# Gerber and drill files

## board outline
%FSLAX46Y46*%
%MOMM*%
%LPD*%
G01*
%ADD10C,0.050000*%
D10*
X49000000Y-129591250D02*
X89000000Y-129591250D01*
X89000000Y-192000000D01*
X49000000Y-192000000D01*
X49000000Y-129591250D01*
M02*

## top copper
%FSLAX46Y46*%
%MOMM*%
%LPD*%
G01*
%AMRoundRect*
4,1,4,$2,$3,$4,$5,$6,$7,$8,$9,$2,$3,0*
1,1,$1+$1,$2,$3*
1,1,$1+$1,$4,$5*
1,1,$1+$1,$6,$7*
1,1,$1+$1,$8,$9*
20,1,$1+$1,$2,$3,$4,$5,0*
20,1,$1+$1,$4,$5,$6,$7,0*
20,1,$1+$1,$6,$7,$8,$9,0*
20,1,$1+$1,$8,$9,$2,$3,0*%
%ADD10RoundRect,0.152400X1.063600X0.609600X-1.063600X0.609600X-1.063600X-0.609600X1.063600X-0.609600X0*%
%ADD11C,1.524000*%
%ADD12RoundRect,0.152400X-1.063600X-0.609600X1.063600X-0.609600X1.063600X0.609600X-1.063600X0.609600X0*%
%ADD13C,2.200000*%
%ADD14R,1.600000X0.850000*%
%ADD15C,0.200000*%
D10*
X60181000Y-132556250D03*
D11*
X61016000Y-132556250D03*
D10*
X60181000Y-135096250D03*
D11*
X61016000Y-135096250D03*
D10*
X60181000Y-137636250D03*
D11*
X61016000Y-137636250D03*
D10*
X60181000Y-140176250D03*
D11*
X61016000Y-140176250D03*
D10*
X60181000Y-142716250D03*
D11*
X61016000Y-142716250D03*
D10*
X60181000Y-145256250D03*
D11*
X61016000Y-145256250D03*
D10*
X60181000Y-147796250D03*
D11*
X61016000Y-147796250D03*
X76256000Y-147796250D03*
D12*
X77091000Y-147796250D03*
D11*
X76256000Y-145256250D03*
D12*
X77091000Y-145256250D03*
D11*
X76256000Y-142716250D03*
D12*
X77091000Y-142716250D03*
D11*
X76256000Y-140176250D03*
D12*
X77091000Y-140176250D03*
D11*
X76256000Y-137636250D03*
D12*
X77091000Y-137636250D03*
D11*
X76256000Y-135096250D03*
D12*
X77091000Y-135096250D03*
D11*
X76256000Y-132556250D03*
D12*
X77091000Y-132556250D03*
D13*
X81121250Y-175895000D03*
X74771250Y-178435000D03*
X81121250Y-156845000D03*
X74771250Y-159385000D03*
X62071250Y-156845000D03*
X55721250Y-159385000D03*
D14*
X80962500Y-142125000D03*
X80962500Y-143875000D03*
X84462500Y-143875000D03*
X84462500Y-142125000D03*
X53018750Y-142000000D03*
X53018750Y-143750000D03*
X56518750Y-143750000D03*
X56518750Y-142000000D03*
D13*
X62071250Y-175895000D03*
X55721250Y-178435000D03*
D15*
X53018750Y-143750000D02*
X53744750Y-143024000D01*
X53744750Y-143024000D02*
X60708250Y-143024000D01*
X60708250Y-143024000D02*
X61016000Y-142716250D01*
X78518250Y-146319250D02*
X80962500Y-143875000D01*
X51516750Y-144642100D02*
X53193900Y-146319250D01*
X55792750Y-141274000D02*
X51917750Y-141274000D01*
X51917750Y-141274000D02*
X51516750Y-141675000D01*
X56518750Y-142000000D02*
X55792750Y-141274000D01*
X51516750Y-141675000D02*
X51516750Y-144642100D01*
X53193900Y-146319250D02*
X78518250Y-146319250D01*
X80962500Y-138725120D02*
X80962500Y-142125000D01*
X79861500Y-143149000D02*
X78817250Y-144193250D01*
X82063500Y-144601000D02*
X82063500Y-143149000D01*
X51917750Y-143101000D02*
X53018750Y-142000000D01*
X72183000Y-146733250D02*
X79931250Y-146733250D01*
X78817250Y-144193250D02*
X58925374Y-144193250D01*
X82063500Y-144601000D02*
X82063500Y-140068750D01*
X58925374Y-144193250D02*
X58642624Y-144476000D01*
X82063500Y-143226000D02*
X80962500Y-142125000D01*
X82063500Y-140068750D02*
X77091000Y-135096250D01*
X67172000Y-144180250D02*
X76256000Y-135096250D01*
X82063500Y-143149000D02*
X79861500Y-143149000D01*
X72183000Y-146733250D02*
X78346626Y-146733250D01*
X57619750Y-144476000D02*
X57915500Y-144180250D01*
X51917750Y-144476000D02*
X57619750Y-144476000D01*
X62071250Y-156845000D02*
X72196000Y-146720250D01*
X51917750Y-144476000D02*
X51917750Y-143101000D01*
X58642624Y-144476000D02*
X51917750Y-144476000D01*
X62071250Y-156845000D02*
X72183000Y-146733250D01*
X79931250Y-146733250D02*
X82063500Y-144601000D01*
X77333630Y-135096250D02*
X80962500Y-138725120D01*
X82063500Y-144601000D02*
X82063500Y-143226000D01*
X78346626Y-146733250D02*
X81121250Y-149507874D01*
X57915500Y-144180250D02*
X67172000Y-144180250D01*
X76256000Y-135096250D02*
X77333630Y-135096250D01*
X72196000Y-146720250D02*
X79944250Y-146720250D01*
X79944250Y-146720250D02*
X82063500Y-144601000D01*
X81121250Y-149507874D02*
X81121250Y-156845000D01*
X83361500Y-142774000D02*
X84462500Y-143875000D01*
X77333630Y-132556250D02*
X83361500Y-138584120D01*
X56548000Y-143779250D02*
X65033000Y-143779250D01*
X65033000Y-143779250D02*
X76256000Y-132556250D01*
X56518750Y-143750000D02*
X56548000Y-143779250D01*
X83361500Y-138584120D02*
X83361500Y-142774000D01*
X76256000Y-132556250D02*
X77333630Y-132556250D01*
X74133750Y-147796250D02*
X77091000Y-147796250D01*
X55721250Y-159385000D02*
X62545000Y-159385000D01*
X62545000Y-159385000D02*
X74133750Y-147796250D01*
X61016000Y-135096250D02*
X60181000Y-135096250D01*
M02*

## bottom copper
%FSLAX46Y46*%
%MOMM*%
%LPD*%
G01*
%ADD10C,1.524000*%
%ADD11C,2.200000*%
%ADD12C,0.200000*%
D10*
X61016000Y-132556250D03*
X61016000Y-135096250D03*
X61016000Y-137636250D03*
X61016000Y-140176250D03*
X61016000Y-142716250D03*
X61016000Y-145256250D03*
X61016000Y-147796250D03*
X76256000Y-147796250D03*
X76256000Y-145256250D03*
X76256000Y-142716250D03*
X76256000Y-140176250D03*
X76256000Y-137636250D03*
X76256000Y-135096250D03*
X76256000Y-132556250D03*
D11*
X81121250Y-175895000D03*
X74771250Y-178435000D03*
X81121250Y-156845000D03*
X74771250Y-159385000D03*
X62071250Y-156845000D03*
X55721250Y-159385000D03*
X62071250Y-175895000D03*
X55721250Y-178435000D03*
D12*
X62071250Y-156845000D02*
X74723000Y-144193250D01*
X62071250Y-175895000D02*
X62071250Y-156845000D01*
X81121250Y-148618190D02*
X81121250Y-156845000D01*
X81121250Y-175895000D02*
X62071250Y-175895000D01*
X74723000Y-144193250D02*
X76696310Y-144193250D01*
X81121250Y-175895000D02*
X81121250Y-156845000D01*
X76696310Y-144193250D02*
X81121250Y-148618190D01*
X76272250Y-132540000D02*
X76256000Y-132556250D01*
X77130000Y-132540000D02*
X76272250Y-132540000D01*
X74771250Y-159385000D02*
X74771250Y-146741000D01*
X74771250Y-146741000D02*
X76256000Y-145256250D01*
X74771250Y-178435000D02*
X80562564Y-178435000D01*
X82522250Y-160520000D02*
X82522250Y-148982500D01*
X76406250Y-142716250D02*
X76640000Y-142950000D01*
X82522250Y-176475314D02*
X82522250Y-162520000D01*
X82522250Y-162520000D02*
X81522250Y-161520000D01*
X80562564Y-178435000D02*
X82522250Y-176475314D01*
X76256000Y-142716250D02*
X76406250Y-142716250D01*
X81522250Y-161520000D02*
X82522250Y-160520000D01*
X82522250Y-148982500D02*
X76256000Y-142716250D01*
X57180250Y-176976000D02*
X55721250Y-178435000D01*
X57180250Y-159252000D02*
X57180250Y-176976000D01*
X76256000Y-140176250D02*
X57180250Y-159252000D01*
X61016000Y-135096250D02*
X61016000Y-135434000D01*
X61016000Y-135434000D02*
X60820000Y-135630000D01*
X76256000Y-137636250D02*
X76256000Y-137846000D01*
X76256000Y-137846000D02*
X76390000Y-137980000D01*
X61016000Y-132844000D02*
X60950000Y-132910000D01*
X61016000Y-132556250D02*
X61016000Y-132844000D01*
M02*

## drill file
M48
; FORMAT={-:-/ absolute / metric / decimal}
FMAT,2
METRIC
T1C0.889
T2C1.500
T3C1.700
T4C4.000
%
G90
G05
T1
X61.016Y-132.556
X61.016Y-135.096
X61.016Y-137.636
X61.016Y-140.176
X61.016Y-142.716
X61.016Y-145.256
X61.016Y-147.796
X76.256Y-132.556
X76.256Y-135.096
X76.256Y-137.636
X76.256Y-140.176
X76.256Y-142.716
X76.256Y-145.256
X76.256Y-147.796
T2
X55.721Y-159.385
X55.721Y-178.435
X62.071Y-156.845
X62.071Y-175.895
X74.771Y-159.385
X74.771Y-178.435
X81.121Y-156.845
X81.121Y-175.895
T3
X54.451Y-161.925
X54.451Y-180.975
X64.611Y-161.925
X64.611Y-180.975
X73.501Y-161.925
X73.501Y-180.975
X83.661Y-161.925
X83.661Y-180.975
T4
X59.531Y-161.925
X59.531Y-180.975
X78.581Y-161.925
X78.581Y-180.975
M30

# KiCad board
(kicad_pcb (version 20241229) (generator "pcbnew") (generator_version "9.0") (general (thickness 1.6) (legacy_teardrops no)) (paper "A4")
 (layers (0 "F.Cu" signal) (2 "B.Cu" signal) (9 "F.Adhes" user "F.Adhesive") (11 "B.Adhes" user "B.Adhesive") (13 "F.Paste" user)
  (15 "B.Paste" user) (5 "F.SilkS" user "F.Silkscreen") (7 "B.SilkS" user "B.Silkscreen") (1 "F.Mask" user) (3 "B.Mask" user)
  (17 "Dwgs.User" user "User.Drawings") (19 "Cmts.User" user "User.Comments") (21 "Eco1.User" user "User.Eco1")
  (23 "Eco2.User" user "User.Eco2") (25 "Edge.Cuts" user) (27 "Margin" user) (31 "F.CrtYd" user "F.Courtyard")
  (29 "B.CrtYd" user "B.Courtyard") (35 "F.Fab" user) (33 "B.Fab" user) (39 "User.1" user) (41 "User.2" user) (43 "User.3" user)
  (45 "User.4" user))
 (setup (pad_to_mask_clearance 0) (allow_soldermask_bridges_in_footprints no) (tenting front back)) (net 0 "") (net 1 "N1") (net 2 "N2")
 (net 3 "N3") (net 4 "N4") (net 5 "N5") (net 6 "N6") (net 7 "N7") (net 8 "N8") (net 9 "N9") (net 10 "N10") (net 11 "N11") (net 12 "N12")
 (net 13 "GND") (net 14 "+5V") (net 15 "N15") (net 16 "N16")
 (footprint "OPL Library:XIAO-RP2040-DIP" (layer "F.Cu") (at 68.636 140.17625)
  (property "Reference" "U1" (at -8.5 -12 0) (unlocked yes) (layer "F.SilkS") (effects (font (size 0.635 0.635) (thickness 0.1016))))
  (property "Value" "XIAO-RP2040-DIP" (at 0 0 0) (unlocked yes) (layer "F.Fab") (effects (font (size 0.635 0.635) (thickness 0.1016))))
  (pad "1" smd roundrect (at -8.455 -7.62 180) (size 2.432 1.524) (layers "F.Cu" "F.Mask") (roundrect_rratio 0.1) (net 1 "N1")
   (thermal_bridge_angle 45))
  (pad "1" thru_hole circle (at -7.62 -7.62 180) (size 1.524 1.524) (drill 0.889) (layers "*.Cu" "*.Mask") (remove_unused_layers no)
   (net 1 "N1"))
  (pad "2" smd roundrect (at -8.455 -5.08 180) (size 2.432 1.524) (layers "F.Cu" "F.Mask") (roundrect_rratio 0.1) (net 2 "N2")
   (thermal_bridge_angle 45))
  (pad "2" thru_hole circle (at -7.62 -5.08 180) (size 1.524 1.524) (drill 0.889) (layers "*.Cu" "*.Mask") (remove_unused_layers no)
   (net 2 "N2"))
  (pad "3" smd roundrect (at -8.455 -2.54 180) (size 2.432 1.524) (layers "F.Cu" "F.Mask") (roundrect_rratio 0.1) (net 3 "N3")
   (thermal_bridge_angle 45))
  (pad "3" thru_hole circle (at -7.62 -2.54 180) (size 1.524 1.524) (drill 0.889) (layers "*.Cu" "*.Mask") (remove_unused_layers no)
   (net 3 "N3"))
  (pad "4" smd roundrect (at -8.455 0 180) (size 2.432 1.524) (layers "F.Cu" "F.Mask") (roundrect_rratio 0.1) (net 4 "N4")
   (thermal_bridge_angle 45))
  (pad "4" thru_hole circle (at -7.62 0 180) (size 1.524 1.524) (drill 0.889) (layers "*.Cu" "*.Mask") (remove_unused_layers no)
   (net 4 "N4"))
  (pad "5" smd roundrect (at -8.455 2.54 180) (size 2.432 1.524) (layers "F.Cu" "F.Mask") (roundrect_rratio 0.1) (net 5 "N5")
   (thermal_bridge_angle 45))
  (pad "5" thru_hole circle (at -7.62 2.54 180) (size 1.524 1.524) (drill 0.889) (layers "*.Cu" "*.Mask") (remove_unused_layers no)
   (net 5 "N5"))
  (pad "6" smd roundrect (at -8.455 5.08 180) (size 2.432 1.524) (layers "F.Cu" "F.Mask") (roundrect_rratio 0.1) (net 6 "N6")
   (thermal_bridge_angle 45))
  (pad "6" thru_hole circle (at -7.62 5.08 180) (size 1.524 1.524) (drill 0.889) (layers "*.Cu" "*.Mask") (remove_unused_layers no)
   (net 6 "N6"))
  (pad "7" smd roundrect (at -8.455 7.62 180) (size 2.432 1.524) (layers "F.Cu" "F.Mask") (roundrect_rratio 0.1) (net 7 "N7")
   (thermal_bridge_angle 45))
  (pad "7" thru_hole circle (at -7.62 7.62 180) (size 1.524 1.524) (drill 0.889) (layers "*.Cu" "*.Mask") (remove_unused_layers no)
   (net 7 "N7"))
  (pad "8" thru_hole circle (at 7.62 7.62) (size 1.524 1.524) (drill 0.889) (layers "*.Cu" "*.Mask") (remove_unused_layers no) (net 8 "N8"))
  (pad "8" smd roundrect (at 8.455 7.62) (size 2.432 1.524) (layers "F.Cu" "F.Mask") (roundrect_rratio 0.1) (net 8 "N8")
   (thermal_bridge_angle 45))
  (pad "9" thru_hole circle (at 7.62 5.08) (size 1.524 1.524) (drill 0.889) (layers "*.Cu" "*.Mask") (remove_unused_layers no) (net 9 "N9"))
  (pad "9" smd roundrect (at 8.455 5.08) (size 2.432 1.524) (layers "F.Cu" "F.Mask") (roundrect_rratio 0.1) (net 9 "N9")
   (thermal_bridge_angle 45))
  (pad "10" thru_hole circle (at 7.62 2.54) (size 1.524 1.524) (drill 0.889) (layers "*.Cu" "*.Mask") (remove_unused_layers no)
   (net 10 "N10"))
  (pad "10" smd roundrect (at 8.455 2.54) (size 2.432 1.524) (layers "F.Cu" "F.Mask") (roundrect_rratio 0.1) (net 10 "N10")
   (thermal_bridge_angle 45))
  (pad "11" thru_hole circle (at 7.62 0) (size 1.524 1.524) (drill 0.889) (layers "*.Cu" "*.Mask") (remove_unused_layers no) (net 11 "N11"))
  (pad "11" smd roundrect (at 8.455 0) (size 2.432 1.524) (layers "F.Cu" "F.Mask") (roundrect_rratio 0.1) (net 11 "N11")
   (thermal_bridge_angle 45))
  (pad "12" thru_hole circle (at 7.62 -2.54) (size 1.524 1.524) (drill 0.889) (layers "*.Cu" "*.Mask") (remove_unused_layers no)
   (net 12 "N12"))
  (pad "12" smd roundrect (at 8.455 -2.54) (size 2.432 1.524) (layers "F.Cu" "F.Mask") (roundrect_rratio 0.1) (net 12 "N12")
   (thermal_bridge_angle 45))
  (pad "13" thru_hole circle (at 7.62 -5.08) (size 1.524 1.524) (drill 0.889) (layers "*.Cu" "*.Mask") (remove_unused_layers no)
   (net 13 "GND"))
  (pad "13" smd roundrect (at 8.455 -5.08) (size 2.432 1.524) (layers "F.Cu" "F.Mask") (roundrect_rratio 0.1) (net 13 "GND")
   (thermal_bridge_angle 45))
  (pad "14" thru_hole circle (at 7.62 -7.62) (size 1.524 1.524) (drill 0.889) (layers "*.Cu" "*.Mask") (remove_unused_layers no)
   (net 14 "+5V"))
  (pad "14" smd roundrect (at 8.455 -7.62) (size 2.432 1.524) (layers "F.Cu" "F.Mask") (roundrect_rratio 0.1) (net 14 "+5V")
   (thermal_bridge_angle 45)))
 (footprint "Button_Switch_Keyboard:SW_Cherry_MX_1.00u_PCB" (layer "F.Cu") (at 81.12125 175.895)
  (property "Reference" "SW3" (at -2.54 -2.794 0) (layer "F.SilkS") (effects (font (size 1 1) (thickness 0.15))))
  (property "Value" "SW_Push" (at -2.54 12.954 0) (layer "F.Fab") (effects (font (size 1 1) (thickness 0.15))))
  (pad "" np_thru_hole circle (at -7.62 5.08) (size 1.7 1.7) (drill 1.7) (layers "*.Cu" "*.Mask"))
  (pad "" np_thru_hole circle (at -2.54 5.08) (size 4 4) (drill 4) (layers "*.Cu" "*.Mask"))
  (pad "" np_thru_hole circle (at 2.54 5.08) (size 1.7 1.7) (drill 1.7) (layers "*.Cu" "*.Mask"))
  (pad "1" thru_hole circle (at 0 0) (size 2.2 2.2) (drill 1.5) (layers "*.Cu" "*.Mask") (remove_unused_layers no) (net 13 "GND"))
  (pad "2" thru_hole circle (at -6.35 2.54) (size 2.2 2.2) (drill 1.5) (layers "*.Cu" "*.Mask") (remove_unused_layers no) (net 10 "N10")))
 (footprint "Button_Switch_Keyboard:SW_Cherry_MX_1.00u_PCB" (layer "F.Cu") (at 81.12125 156.845)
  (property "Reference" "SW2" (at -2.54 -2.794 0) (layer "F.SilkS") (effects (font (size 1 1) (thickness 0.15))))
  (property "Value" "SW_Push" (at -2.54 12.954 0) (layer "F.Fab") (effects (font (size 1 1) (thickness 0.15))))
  (pad "" np_thru_hole circle (at -7.62 5.08) (size 1.7 1.7) (drill 1.7) (layers "*.Cu" "*.Mask"))
  (pad "" np_thru_hole circle (at -2.54 5.08) (size 4 4) (drill 4) (layers "*.Cu" "*.Mask"))
  (pad "" np_thru_hole circle (at 2.54 5.08) (size 1.7 1.7) (drill 1.7) (layers "*.Cu" "*.Mask"))
  (pad "1" thru_hole circle (at 0 0) (size 2.2 2.2) (drill 1.5) (layers "*.Cu" "*.Mask") (remove_unused_layers no) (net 13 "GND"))
  (pad "2" thru_hole circle (at -6.35 2.54) (size 2.2 2.2) (drill 1.5) (layers "*.Cu" "*.Mask") (remove_unused_layers no) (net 9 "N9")))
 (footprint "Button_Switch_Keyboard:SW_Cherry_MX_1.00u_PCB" (layer "F.Cu") (at 62.07125 156.845)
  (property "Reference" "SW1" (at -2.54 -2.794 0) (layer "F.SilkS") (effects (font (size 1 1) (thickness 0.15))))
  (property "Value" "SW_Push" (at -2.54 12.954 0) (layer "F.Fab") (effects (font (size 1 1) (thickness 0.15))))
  (pad "" np_thru_hole circle (at -7.62 5.08) (size 1.7 1.7) (drill 1.7) (layers "*.Cu" "*.Mask"))
  (pad "" np_thru_hole circle (at -2.54 5.08) (size 4 4) (drill 4) (layers "*.Cu" "*.Mask"))
  (pad "" np_thru_hole circle (at 2.54 5.08) (size 1.7 1.7) (drill 1.7) (layers "*.Cu" "*.Mask"))
  (pad "1" thru_hole circle (at 0 0) (size 2.2 2.2) (drill 1.5) (layers "*.Cu" "*.Mask") (remove_unused_layers no) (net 13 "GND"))
  (pad "2" thru_hole circle (at -6.35 2.54) (size 2.2 2.2) (drill 1.5) (layers "*.Cu" "*.Mask") (remove_unused_layers no) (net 8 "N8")))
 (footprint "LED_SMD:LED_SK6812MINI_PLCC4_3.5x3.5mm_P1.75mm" (layer "F.Cu") (at 82.7125 143)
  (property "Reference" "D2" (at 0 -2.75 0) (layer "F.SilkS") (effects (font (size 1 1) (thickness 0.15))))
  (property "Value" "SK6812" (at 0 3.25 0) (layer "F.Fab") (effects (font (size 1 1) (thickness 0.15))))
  (pad "1" smd rect (at -1.75 -0.875) (size 1.6 0.85) (layers "F.Cu" "F.Mask" "F.Paste") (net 13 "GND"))
  (pad "2" smd rect (at -1.75 0.875) (size 1.6 0.85) (layers "F.Cu" "F.Mask" "F.Paste") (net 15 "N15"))
  (pad "3" smd rect (at 1.75 0.875) (size 1.6 0.85) (layers "F.Cu" "F.Mask" "F.Paste") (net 14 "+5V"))
  (pad "4" smd rect (at 1.75 -0.875) (size 1.6 0.85) (layers "F.Cu" "F.Mask" "F.Paste") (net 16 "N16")))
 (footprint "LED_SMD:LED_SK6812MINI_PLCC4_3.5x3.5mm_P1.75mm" (layer "F.Cu") (at 54.76875 142.875)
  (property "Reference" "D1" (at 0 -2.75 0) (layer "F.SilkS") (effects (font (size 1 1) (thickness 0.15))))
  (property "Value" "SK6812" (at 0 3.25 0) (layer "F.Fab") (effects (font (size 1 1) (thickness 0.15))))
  (pad "1" smd rect (at -1.75 -0.875) (size 1.6 0.85) (layers "F.Cu" "F.Mask" "F.Paste") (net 13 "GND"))
  (pad "2" smd rect (at -1.75 0.875) (size 1.6 0.85) (layers "F.Cu" "F.Mask" "F.Paste") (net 5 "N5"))
  (pad "3" smd rect (at 1.75 0.875) (size 1.6 0.85) (layers "F.Cu" "F.Mask" "F.Paste") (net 14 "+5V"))
  (pad "4" smd rect (at 1.75 -0.875) (size 1.6 0.85) (layers "F.Cu" "F.Mask" "F.Paste") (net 15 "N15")))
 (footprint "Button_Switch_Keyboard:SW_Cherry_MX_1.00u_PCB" (layer "F.Cu") (at 62.07125 175.895)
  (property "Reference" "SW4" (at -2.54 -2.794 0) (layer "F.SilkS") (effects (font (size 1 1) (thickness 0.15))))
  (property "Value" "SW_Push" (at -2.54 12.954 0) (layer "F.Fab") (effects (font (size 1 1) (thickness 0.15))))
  (pad "" np_thru_hole circle (at -7.62 5.08) (size 1.7 1.7) (drill 1.7) (layers "*.Cu" "*.Mask"))
  (pad "" np_thru_hole circle (at -2.54 5.08) (size 4 4) (drill 4) (layers "*.Cu" "*.Mask"))
  (pad "" np_thru_hole circle (at 2.54 5.08) (size 1.7 1.7) (drill 1.7) (layers "*.Cu" "*.Mask"))
  (pad "1" thru_hole circle (at 0 0) (size 2.2 2.2) (drill 1.5) (layers "*.Cu" "*.Mask") (remove_unused_layers no) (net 13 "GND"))
  (pad "2" thru_hole circle (at -6.35 2.54) (size 2.2 2.2) (drill 1.5) (layers "*.Cu" "*.Mask") (remove_unused_layers no) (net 11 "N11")))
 (gr_rect (start 49 129.59125) (end 89 192) (stroke (width 0.05) (type default)) (fill no) (layer "Edge.Cuts"))
 (segment (start 53.01875 143.75) (end 53.74475 143.024) (width 0.2) (layer "F.Cu") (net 5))
 (segment (start 53.74475 143.024) (end 60.70825 143.024) (width 0.2) (layer "F.Cu") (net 5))
 (segment (start 60.70825 143.024) (end 61.016 142.71625) (width 0.2) (layer "F.Cu") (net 5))
 (segment (start 78.51825 146.31925) (end 80.9625 143.875) (width 0.2) (layer "F.Cu") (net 15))
 (segment (start 51.51675 144.6421) (end 53.1939 146.31925) (width 0.2) (layer "F.Cu") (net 15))
 (segment (start 55.79275 141.274) (end 51.91775 141.274) (width 0.2) (layer "F.Cu") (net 15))
 (segment (start 51.91775 141.274) (end 51.51675 141.675) (width 0.2) (layer "F.Cu") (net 15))
 (segment (start 56.51875 142) (end 55.79275 141.274) (width 0.2) (layer "F.Cu") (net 15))
 (segment (start 51.51675 141.675) (end 51.51675 144.6421) (width 0.2) (layer "F.Cu") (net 15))
 (segment (start 53.1939 146.31925) (end 78.51825 146.31925) (width 0.2) (layer "F.Cu") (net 15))
 (segment (start 80.9625 138.72512) (end 80.9625 142.125) (width 0.2) (layer "F.Cu") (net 13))
 (segment (start 79.8615 143.149) (end 78.81725 144.19325) (width 0.2) (layer "F.Cu") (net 13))
 (segment (start 82.0635 144.601) (end 82.0635 143.149) (width 0.2) (layer "F.Cu") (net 13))
 (segment (start 51.91775 143.101) (end 53.01875 142) (width 0.2) (layer "F.Cu") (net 13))
 (segment (start 72.183 146.73325) (end 79.93125 146.73325) (width 0.2) (layer "F.Cu") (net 13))
 (segment (start 78.81725 144.19325) (end 58.925374 144.19325) (width 0.2) (layer "F.Cu") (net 13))
 (segment (start 82.0635 144.601) (end 82.0635 140.06875) (width 0.2) (layer "F.Cu") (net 13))
 (segment (start 58.925374 144.19325) (end 58.642624 144.476) (width 0.2) (layer "F.Cu") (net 13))
 (segment (start 82.0635 143.226) (end 80.9625 142.125) (width 0.2) (layer "F.Cu") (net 13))
 (segment (start 82.0635 140.06875) (end 77.091 135.09625) (width 0.2) (layer "F.Cu") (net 13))
 (segment (start 67.172 144.18025) (end 76.256 135.09625) (width 0.2) (layer "F.Cu") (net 13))
 (segment (start 82.0635 143.149) (end 79.8615 143.149) (width 0.2) (layer "F.Cu") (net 13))
 (segment (start 72.183 146.73325) (end 78.346626 146.73325) (width 0.2) (layer "F.Cu") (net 13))
 (segment (start 57.61975 144.476) (end 57.9155 144.18025) (width 0.2) (layer "F.Cu") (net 13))
 (segment (start 51.91775 144.476) (end 57.61975 144.476) (width 0.2) (layer "F.Cu") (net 13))
 (segment (start 62.07125 156.845) (end 72.196 146.72025) (width 0.2) (layer "F.Cu") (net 13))
 (segment (start 51.91775 144.476) (end 51.91775 143.101) (width 0.2) (layer "F.Cu") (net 13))
 (segment (start 58.642624 144.476) (end 51.91775 144.476) (width 0.2) (layer "F.Cu") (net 13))
 (segment (start 62.07125 156.845) (end 72.183 146.73325) (width 0.2) (layer "F.Cu") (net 13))
 (segment (start 79.93125 146.73325) (end 82.0635 144.601) (width 0.2) (layer "F.Cu") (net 13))
 (segment (start 77.33363 135.09625) (end 80.9625 138.72512) (width 0.2) (layer "F.Cu") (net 13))
 (segment (start 82.0635 144.601) (end 82.0635 143.226) (width 0.2) (layer "F.Cu") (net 13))
 (segment (start 78.346626 146.73325) (end 81.12125 149.507874) (width 0.2) (layer "F.Cu") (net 13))
 (segment (start 57.9155 144.18025) (end 67.172 144.18025) (width 0.2) (layer "F.Cu") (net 13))
 (segment (start 76.256 135.09625) (end 77.33363 135.09625) (width 0.2) (layer "F.Cu") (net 13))
 (segment (start 72.196 146.72025) (end 79.94425 146.72025) (width 0.2) (layer "F.Cu") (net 13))
 (segment (start 79.94425 146.72025) (end 82.0635 144.601) (width 0.2) (layer "F.Cu") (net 13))
 (segment (start 81.12125 149.507874) (end 81.12125 156.845) (width 0.2) (layer "F.Cu") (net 13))
 (segment (start 62.07125 156.845) (end 74.723 144.19325) (width 0.2) (layer "B.Cu") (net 13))
 (segment (start 62.07125 175.895) (end 62.07125 156.845) (width 0.2) (layer "B.Cu") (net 13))
 (segment (start 81.12125 148.61819) (end 81.12125 156.845) (width 0.2) (layer "B.Cu") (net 13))
 (segment (start 81.12125 175.895) (end 62.07125 175.895) (width 0.2) (layer "B.Cu") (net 13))
 (segment (start 74.723 144.19325) (end 76.69631 144.19325) (width 0.2) (layer "B.Cu") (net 13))
 (segment (start 81.12125 175.895) (end 81.12125 156.845) (width 0.2) (layer "B.Cu") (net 13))
 (segment (start 76.69631 144.19325) (end 81.12125 148.61819) (width 0.2) (layer "B.Cu") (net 13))
 (segment (start 83.3615 142.774) (end 84.4625 143.875) (width 0.2) (layer "F.Cu") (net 14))
 (segment (start 77.33363 132.55625) (end 83.3615 138.58412) (width 0.2) (layer "F.Cu") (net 14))
 (segment (start 56.548 143.77925) (end 65.033 143.77925) (width 0.2) (layer "F.Cu") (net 14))
 (segment (start 65.033 143.77925) (end 76.256 132.55625) (width 0.2) (layer "F.Cu") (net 14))
 (segment (start 56.51875 143.75) (end 56.548 143.77925) (width 0.2) (layer "F.Cu") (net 14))
 (segment (start 83.3615 138.58412) (end 83.3615 142.774) (width 0.2) (layer "F.Cu") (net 14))
 (segment (start 76.256 132.55625) (end 77.33363 132.55625) (width 0.2) (layer "F.Cu") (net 14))
 (segment (start 76.27225 132.54) (end 76.256 132.55625) (width 0.2) (layer "B.Cu") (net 14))
 (segment (start 77.13 132.54) (end 76.27225 132.54) (width 0.2) (layer "B.Cu") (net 14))
 (segment (start 74.13375 147.79625) (end 77.091 147.79625) (width 0.2) (layer "F.Cu") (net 8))
 (segment (start 55.72125 159.385) (end 62.545 159.385) (width 0.2) (layer "F.Cu") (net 8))
 (segment (start 62.545 159.385) (end 74.13375 147.79625) (width 0.2) (layer "F.Cu") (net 8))
 (segment (start 74.77125 159.385) (end 74.77125 146.741) (width 0.2) (layer "B.Cu") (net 9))
 (segment (start 74.77125 146.741) (end 76.256 145.25625) (width 0.2) (layer "B.Cu") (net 9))
 (segment (start 74.77125 178.435) (end 80.562564 178.435) (width 0.2) (layer "B.Cu") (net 10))
 (segment (start 82.52225 160.52) (end 82.52225 148.9825) (width 0.2) (layer "B.Cu") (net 10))
 (segment (start 76.40625 142.71625) (end 76.64 142.95) (width 0.2) (layer "B.Cu") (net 10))
 (segment (start 82.52225 176.475314) (end 82.52225 162.52) (width 0.2) (layer "B.Cu") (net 10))
 (segment (start 82.52225 162.52) (end 81.52225 161.52) (width 0.2) (layer "B.Cu") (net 10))
 (segment (start 80.562564 178.435) (end 82.52225 176.475314) (width 0.2) (layer "B.Cu") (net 10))
 (segment (start 76.256 142.71625) (end 76.40625 142.71625) (width 0.2) (layer "B.Cu") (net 10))
 (segment (start 81.52225 161.52) (end 82.52225 160.52) (width 0.2) (layer "B.Cu") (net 10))
 (segment (start 82.52225 148.9825) (end 76.256 142.71625) (width 0.2) (layer "B.Cu") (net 10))
 (segment (start 57.18025 176.976) (end 55.72125 178.435) (width 0.2) (layer "B.Cu") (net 11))
 (segment (start 57.18025 159.252) (end 57.18025 176.976) (width 0.2) (layer "B.Cu") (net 11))
 (segment (start 76.256 140.17625) (end 57.18025 159.252) (width 0.2) (layer "B.Cu") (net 11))
 (segment (start 61.016 135.09625) (end 60.181 135.09625) (width 0.2) (layer "F.Cu") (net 2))
 (segment (start 61.016 135.09625) (end 61.016 135.434) (width 0.2) (layer "B.Cu") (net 2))
 (segment (start 61.016 135.434) (end 60.82 135.63) (width 0.2) (layer "B.Cu") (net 2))
 (segment (start 76.256 137.63625) (end 76.256 137.846) (width 0.2) (layer "B.Cu") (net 12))
 (segment (start 76.256 137.846) (end 76.39 137.98) (width 0.2) (layer "B.Cu") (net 12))
 (segment (start 61.016 132.844) (end 60.95 132.91) (width 0.2) (layer "B.Cu") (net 1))
 (segment (start 61.016 132.55625) (end 61.016 132.844) (width 0.2) (layer "B.Cu") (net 1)))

